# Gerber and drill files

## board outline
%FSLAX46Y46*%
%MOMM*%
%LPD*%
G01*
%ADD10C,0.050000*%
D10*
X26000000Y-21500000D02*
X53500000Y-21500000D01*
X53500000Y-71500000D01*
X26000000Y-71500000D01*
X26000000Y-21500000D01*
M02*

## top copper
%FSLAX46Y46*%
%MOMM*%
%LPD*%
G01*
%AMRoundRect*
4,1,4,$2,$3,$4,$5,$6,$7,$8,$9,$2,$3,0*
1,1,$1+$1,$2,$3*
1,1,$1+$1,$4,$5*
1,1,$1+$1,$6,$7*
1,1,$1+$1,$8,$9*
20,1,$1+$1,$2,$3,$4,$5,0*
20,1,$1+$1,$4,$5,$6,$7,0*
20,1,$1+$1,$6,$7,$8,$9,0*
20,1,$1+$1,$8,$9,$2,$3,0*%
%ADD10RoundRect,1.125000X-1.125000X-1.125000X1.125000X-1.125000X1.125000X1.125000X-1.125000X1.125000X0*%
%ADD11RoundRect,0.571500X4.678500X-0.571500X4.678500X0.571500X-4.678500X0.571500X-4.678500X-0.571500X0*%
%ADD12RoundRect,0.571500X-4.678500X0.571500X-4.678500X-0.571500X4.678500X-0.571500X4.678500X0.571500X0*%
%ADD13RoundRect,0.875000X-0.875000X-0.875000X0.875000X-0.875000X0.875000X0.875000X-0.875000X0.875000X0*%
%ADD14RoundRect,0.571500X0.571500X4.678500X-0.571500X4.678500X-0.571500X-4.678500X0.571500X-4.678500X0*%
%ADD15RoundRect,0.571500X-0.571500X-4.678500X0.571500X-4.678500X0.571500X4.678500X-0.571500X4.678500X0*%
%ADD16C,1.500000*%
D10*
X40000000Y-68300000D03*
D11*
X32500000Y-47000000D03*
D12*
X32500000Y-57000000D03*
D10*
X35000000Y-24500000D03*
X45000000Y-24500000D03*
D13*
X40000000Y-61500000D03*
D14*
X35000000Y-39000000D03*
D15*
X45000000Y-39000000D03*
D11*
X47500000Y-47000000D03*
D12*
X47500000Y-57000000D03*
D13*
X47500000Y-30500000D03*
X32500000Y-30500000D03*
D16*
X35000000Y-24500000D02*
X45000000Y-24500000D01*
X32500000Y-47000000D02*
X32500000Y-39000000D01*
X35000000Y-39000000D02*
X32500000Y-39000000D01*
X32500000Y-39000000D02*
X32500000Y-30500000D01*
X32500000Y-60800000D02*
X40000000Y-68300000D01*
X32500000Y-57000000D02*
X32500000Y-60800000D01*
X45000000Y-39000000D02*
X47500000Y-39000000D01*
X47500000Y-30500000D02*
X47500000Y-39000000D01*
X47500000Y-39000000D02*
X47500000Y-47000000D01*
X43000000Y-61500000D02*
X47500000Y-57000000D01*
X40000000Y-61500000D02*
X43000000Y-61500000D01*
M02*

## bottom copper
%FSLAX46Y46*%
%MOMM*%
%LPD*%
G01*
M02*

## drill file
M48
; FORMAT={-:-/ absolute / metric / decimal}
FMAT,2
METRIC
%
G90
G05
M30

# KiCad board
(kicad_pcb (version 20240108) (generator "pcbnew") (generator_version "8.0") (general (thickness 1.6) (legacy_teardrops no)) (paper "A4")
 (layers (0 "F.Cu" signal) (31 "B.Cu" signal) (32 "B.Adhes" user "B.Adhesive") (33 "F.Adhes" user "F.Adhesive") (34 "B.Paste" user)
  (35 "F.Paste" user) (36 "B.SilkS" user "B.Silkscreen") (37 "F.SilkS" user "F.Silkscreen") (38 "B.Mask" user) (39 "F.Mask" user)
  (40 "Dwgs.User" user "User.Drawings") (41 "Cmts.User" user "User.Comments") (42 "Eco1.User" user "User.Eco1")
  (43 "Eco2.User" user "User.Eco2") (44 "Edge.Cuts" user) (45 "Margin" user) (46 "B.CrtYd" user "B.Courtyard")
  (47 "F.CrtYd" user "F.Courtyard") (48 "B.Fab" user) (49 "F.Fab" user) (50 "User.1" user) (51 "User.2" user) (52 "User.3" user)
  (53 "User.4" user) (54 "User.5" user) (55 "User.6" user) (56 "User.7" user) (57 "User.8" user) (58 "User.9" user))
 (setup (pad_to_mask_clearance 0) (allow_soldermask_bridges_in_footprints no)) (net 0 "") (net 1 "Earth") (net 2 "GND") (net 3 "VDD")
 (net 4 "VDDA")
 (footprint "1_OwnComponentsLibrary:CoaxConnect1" (layer "F.Cu") (at 40 68.3)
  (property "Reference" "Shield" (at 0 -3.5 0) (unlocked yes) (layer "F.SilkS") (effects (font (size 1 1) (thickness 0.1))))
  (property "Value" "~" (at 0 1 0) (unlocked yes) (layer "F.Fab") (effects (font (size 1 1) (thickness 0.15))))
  (pad "1" smd roundrect (at 0 0) (size 4.5 4.5) (layers "F.Cu" "F.Paste" "F.Mask") (roundrect_rratio 0.25) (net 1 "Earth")
   (thermal_bridge_angle 45)))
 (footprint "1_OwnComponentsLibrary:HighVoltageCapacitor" (layer "F.Cu") (at 32.5 52 -90)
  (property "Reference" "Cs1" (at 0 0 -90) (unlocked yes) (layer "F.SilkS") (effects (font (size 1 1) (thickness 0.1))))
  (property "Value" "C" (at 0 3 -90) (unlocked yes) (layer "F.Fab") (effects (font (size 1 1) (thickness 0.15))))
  (pad "1" smd roundrect (at -5 0 90) (size 2.286 10.5) (layers "F.Cu" "F.Paste" "F.Mask") (roundrect_rratio 0.25) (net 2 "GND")
   (thermal_bridge_angle 45))
  (pad "2" smd roundrect (at 5 0 270) (size 2.286 10.5) (layers "F.Cu" "F.Paste" "F.Mask") (roundrect_rratio 0.25) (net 1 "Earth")
   (thermal_bridge_angle 45)))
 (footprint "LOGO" (layer "F.Cu") (at 32 68.563205)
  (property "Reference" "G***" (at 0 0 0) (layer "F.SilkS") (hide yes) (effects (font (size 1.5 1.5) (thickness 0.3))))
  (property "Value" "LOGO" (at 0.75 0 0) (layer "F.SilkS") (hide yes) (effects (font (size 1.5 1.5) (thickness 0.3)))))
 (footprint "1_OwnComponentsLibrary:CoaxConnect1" (layer "F.Cu") (at 35 24.5)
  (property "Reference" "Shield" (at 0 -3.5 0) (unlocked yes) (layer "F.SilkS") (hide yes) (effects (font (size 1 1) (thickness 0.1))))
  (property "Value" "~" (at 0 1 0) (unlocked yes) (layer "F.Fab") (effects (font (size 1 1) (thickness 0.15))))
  (pad "1" smd roundrect (at 0 0) (size 4.5 4.5) (layers "F.Cu" "F.Paste" "F.Mask") (roundrect_rratio 0.25) (thermal_bridge_angle 45)))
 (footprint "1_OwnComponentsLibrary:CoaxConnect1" (layer "F.Cu") (at 45 24.5)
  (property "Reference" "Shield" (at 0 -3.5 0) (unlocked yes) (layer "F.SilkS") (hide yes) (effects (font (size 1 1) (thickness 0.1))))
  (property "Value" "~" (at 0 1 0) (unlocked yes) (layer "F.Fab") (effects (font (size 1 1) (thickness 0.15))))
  (pad "1" smd roundrect (at 0 0) (size 4.5 4.5) (layers "F.Cu" "F.Paste" "F.Mask") (roundrect_rratio 0.25) (thermal_bridge_angle 45)))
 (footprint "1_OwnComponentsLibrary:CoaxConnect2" (layer "F.Cu") (at 40 61.5)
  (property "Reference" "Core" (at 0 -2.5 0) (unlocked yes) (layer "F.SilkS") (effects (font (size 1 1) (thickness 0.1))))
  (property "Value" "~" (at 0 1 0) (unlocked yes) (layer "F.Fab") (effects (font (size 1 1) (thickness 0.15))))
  (pad "1" smd roundrect (at 0 0) (size 3.5 3.5) (layers "F.Cu" "F.Paste" "F.Mask") (roundrect_rratio 0.25) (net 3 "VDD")
   (thermal_bridge_angle 45)))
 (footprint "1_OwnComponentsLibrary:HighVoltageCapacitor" (layer "F.Cu") (at 40 39)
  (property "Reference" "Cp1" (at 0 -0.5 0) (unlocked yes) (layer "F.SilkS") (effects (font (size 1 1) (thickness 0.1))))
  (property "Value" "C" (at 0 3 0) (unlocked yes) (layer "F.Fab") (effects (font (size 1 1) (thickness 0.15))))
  (pad "1" smd roundrect (at -5 0 180) (size 2.286 10.5) (layers "F.Cu" "F.Paste" "F.Mask") (roundrect_rratio 0.25) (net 2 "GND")
   (thermal_bridge_angle 45))
  (pad "2" smd roundrect (at 5 0) (size 2.286 10.5) (layers "F.Cu" "F.Paste" "F.Mask") (roundrect_rratio 0.25) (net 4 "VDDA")
   (thermal_bridge_angle 45)))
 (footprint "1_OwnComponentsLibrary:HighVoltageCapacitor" (layer "F.Cu") (at 47.5 52 -90)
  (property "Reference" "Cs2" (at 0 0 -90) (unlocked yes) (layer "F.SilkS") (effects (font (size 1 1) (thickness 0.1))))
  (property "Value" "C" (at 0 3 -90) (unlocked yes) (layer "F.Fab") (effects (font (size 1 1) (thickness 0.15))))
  (pad "1" smd roundrect (at -5 0 90) (size 2.286 10.5) (layers "F.Cu" "F.Paste" "F.Mask") (roundrect_rratio 0.25) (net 4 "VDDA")
   (thermal_bridge_angle 45))
  (pad "2" smd roundrect (at 5 0 270) (size 2.286 10.5) (layers "F.Cu" "F.Paste" "F.Mask") (roundrect_rratio 0.25) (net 3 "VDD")
   (thermal_bridge_angle 45)))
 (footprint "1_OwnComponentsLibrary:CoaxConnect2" (layer "F.Cu") (at 47.5 30.5)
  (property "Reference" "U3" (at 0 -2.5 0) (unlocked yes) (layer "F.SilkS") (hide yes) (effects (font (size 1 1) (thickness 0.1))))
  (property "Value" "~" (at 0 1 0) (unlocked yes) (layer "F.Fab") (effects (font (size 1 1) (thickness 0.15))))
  (pad "1" smd roundrect (at 0 0) (size 3.5 3.5) (layers "F.Cu" "F.Paste" "F.Mask") (roundrect_rratio 0.25) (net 4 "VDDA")
   (thermal_bridge_angle 45)))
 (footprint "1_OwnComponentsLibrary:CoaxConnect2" (layer "F.Cu") (at 32.5 30.5)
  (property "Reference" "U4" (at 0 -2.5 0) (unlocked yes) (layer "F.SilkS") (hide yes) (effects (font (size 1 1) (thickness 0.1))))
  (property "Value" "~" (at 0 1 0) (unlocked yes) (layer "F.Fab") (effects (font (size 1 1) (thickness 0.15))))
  (pad "1" smd roundrect (at 0 0) (size 3.5 3.5) (layers "F.Cu" "F.Paste" "F.Mask") (roundrect_rratio 0.25) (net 2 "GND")
   (thermal_bridge_angle 45)))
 (gr_rect (start 26 21.5) (end 53.5 71.5) (stroke (width 0.05) (type default)) (fill none) (layer "Edge.Cuts"))
 (segment (start 35 24.5) (end 45 24.5) (width 1.5) (layer "F.Cu") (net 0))
 (segment (start 32.5 47) (end 32.5 39) (width 1.5) (layer "F.Cu") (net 2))
 (segment (start 35 39) (end 32.5 39) (width 1.5) (layer "F.Cu") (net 2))
 (segment (start 32.5 39) (end 32.5 30.5) (width 1.5) (layer "F.Cu") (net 2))
 (segment (start 32.5 60.8) (end 40 68.3) (width 1.5) (layer "F.Cu") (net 1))
 (segment (start 32.5 57) (end 32.5 60.8) (width 1.5) (layer "F.Cu") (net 1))
 (segment (start 45 39) (end 47.5 39) (width 1.5) (layer "F.Cu") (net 4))
 (segment (start 47.5 30.5) (end 47.5 39) (width 1.5) (layer "F.Cu") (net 4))
 (segment (start 47.5 39) (end 47.5 47) (width 1.5) (layer "F.Cu") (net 4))
 (segment (start 43 61.5) (end 47.5 57) (width 1.5) (layer "F.Cu") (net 3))
 (segment (start 40 61.5) (end 43 61.5) (width 1.5) (layer "F.Cu") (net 3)))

